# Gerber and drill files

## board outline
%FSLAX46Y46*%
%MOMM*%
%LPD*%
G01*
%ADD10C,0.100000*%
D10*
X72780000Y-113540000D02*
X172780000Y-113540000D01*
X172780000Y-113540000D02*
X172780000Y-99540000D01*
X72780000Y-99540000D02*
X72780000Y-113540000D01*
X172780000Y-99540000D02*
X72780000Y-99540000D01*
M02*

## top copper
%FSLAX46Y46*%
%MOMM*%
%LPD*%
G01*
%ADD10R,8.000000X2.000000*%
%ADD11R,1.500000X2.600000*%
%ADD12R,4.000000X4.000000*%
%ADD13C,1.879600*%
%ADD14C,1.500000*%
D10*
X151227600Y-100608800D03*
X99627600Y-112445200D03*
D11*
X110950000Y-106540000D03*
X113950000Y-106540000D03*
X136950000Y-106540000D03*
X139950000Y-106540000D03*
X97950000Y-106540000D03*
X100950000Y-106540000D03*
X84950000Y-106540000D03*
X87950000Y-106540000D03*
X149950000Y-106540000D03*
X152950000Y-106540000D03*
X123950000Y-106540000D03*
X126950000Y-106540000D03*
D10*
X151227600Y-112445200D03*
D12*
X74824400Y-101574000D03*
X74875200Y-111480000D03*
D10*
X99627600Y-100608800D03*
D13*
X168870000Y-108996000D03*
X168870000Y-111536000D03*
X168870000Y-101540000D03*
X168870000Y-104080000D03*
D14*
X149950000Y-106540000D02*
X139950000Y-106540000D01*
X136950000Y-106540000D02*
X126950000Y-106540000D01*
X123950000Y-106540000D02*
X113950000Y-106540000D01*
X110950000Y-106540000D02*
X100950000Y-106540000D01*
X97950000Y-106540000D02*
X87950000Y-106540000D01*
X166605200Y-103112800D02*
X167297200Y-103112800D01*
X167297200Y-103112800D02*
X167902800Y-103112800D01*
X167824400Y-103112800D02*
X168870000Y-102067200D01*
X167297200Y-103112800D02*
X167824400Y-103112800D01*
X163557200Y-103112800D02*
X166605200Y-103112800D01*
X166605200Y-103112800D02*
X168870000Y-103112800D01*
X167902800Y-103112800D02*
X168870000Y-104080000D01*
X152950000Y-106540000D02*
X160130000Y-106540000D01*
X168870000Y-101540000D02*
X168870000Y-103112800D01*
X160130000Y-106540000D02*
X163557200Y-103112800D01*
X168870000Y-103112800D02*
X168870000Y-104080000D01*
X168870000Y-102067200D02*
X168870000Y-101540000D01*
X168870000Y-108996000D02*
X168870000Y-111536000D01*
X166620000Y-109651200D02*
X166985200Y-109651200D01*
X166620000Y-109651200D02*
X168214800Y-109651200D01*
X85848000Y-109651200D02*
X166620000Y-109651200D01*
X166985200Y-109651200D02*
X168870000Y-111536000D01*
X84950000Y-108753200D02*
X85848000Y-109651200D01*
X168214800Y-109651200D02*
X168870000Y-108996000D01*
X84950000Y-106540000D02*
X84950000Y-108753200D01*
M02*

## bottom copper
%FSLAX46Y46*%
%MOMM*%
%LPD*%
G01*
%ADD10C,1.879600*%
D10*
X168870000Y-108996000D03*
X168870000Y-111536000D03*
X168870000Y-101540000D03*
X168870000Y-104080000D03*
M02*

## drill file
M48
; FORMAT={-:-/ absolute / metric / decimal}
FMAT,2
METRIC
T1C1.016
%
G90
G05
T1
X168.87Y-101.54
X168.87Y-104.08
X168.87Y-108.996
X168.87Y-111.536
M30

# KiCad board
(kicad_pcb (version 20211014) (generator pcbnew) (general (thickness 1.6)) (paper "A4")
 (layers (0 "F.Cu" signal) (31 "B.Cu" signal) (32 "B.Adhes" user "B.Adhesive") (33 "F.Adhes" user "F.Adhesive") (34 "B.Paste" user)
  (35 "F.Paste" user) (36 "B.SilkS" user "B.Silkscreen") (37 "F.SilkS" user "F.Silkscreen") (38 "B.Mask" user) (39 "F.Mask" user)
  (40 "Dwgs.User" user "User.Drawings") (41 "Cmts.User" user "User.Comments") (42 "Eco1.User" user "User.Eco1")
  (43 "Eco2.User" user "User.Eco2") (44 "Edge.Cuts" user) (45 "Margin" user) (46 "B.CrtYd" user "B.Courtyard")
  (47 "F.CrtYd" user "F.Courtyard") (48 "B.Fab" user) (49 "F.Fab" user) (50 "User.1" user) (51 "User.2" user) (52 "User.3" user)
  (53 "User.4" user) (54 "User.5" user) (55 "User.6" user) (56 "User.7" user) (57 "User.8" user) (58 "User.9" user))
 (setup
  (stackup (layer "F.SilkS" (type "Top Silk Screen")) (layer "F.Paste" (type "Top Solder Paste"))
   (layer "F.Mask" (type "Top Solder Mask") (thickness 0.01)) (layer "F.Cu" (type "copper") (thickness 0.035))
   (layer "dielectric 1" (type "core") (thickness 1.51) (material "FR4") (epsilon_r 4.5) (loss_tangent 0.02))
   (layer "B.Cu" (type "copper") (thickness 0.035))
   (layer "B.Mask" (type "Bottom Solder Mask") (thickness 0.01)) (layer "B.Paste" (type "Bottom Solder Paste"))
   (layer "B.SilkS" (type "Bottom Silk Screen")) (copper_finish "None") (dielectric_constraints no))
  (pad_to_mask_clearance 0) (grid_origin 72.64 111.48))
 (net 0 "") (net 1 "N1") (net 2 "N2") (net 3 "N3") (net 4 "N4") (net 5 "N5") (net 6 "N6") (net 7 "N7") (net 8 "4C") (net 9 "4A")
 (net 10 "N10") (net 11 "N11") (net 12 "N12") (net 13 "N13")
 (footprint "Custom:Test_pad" (layer "F.Cu") (at 151.2276 100.6088)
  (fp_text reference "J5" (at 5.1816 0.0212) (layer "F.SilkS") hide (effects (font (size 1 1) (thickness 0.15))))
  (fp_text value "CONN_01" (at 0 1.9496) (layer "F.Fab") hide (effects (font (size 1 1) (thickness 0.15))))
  (pad "1" smd rect (at 0 0) (size 8 2) (layers "F.Cu" "F.Mask") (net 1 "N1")))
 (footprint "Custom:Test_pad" (layer "F.Cu") (at 99.6276 112.4452)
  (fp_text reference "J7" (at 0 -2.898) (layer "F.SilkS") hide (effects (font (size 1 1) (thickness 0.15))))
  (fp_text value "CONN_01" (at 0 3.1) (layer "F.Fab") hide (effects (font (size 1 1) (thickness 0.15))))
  (pad "1" smd rect (at 0 0) (size 8 2) (layers "F.Cu" "F.Mask") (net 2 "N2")))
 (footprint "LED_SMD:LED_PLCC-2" (layer "F.Cu") (at 112.45 106.54)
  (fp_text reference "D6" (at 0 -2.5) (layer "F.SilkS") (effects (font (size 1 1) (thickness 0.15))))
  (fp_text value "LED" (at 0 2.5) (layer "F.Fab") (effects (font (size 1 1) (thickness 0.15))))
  (pad "1" smd rect (at -1.5 0) (size 1.5 2.6) (layers "F.Cu" "F.Paste" "F.Mask") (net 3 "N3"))
  (pad "2" smd rect (at 1.5 0) (size 1.5 2.6) (layers "F.Cu" "F.Paste" "F.Mask") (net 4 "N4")))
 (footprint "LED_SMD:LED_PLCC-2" (layer "F.Cu") (at 138.45 106.54)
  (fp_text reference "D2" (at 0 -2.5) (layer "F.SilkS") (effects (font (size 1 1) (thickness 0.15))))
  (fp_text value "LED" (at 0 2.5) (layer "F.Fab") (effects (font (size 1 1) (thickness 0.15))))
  (pad "1" smd rect (at -1.5 0) (size 1.5 2.6) (layers "F.Cu" "F.Paste" "F.Mask") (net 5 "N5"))
  (pad "2" smd rect (at 1.5 0) (size 1.5 2.6) (layers "F.Cu" "F.Paste" "F.Mask") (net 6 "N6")))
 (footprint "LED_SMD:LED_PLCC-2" (layer "F.Cu") (at 99.45 106.54)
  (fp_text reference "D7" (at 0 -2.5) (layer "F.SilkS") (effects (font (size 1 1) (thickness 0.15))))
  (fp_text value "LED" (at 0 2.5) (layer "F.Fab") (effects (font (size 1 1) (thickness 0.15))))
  (pad "1" smd rect (at -1.5 0) (size 1.5 2.6) (layers "F.Cu" "F.Paste" "F.Mask") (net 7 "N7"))
  (pad "2" smd rect (at 1.5 0) (size 1.5 2.6) (layers "F.Cu" "F.Paste" "F.Mask") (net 3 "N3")))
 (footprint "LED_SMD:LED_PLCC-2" (layer "F.Cu") (at 86.45 106.54)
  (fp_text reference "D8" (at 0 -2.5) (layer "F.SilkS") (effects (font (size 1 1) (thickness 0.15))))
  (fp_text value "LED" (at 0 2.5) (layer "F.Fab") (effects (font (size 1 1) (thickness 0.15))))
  (pad "1" smd rect (at -1.5 0) (size 1.5 2.6) (layers "F.Cu" "F.Paste" "F.Mask") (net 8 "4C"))
  (pad "2" smd rect (at 1.5 0) (size 1.5 2.6) (layers "F.Cu" "F.Paste" "F.Mask") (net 7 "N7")))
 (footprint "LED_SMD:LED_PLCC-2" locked (layer "F.Cu") (at 151.45 106.54)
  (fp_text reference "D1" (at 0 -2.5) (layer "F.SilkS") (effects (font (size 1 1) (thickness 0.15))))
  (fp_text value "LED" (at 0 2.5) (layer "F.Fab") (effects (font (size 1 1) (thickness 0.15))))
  (pad "1" smd rect locked (at -1.5 0) (size 1.5 2.6) (layers "F.Cu" "F.Paste" "F.Mask") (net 6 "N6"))
  (pad "2" smd rect locked (at 1.5 0) (size 1.5 2.6) (layers "F.Cu" "F.Paste" "F.Mask") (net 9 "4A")))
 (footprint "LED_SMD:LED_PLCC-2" (layer "F.Cu") (at 125.45 106.54)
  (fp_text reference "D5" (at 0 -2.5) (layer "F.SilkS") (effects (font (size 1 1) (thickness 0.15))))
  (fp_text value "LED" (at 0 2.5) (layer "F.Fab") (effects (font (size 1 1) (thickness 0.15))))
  (pad "1" smd rect (at -1.5 0) (size 1.5 2.6) (layers "F.Cu" "F.Paste" "F.Mask") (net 4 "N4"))
  (pad "2" smd rect (at 1.5 0) (size 1.5 2.6) (layers "F.Cu" "F.Paste" "F.Mask") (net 5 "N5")))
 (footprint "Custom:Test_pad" (layer "F.Cu") (at 151.2276 112.4452)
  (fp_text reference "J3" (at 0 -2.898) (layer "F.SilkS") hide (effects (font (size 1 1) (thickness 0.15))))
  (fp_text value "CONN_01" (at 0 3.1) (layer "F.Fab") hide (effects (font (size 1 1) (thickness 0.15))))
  (pad "1" smd rect (at 0 0) (size 8 2) (layers "F.Cu" "F.Mask") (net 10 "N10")))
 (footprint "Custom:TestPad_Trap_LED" (layer "F.Cu") (at 74.8244 101.574)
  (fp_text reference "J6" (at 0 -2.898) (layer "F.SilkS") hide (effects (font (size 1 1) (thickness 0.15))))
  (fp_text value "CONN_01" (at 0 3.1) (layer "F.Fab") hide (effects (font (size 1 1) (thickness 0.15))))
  (pad "1" smd rect (at 0 0) (size 4 4) (layers "F.Cu" "F.Mask") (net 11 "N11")))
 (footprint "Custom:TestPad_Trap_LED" (layer "F.Cu") (at 74.8752 111.48)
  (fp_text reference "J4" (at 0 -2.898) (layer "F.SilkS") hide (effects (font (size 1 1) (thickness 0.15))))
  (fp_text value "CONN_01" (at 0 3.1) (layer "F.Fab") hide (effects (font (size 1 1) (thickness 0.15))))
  (pad "1" smd rect (at 0 0) (size 4 4) (layers "F.Cu" "F.Mask") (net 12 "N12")))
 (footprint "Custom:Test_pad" (layer "F.Cu") (at 99.6276 100.6088)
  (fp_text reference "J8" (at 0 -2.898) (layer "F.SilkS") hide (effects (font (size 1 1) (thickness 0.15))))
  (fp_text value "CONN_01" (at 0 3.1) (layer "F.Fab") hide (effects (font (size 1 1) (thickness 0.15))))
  (pad "1" smd rect (at 0 0) (size 8 2) (layers "F.Cu" "F.Mask") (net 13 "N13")))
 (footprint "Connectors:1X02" (layer "B.Cu") (at 168.87 108.996 -90)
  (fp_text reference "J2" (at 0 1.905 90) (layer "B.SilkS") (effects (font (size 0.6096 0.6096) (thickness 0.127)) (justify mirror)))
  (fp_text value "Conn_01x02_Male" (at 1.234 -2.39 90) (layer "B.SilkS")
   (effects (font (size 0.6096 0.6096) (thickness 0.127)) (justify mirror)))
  (pad "1" thru_hole circle locked (at 0 0 270) (size 1.8796 1.8796) (drill 1.016) (layers *.Cu *.Mask) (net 8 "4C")
   (solder_mask_margin 0.1016))
  (pad "2" thru_hole circle locked (at 2.54 0 270) (size 1.8796 1.8796) (drill 1.016) (layers *.Cu *.Mask) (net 8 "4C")
   (solder_mask_margin 0.1016)))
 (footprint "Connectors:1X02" (layer "B.Cu") (at 168.87 101.54 -90)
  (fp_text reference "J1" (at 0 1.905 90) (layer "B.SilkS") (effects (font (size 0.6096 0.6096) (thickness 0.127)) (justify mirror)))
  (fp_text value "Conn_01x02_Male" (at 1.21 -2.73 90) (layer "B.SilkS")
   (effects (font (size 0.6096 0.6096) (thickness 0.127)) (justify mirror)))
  (pad "1" thru_hole circle locked (at 0 0 270) (size 1.8796 1.8796) (drill 1.016) (layers *.Cu *.Mask) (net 9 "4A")
   (solder_mask_margin 0.1016))
  (pad "2" thru_hole circle locked (at 2.54 0 270) (size 1.8796 1.8796) (drill 1.016) (layers *.Cu *.Mask) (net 9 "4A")
   (solder_mask_margin 0.1016)))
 (gr_line (start 72.78 113.54) (end 172.78 113.54) (layer "Edge.Cuts") (width 0.1))
 (gr_line (start 172.78 113.54) (end 172.78 99.54) (layer "Edge.Cuts") (width 0.1))
 (gr_line (start 72.78 99.54) (end 72.78 113.54) (layer "Edge.Cuts") (width 0.1))
 (gr_line (start 172.78 99.54) (end 72.78 99.54) (layer "Edge.Cuts") (width 0.1))
 (segment (start 149.95 106.54) (end 139.95 106.54) (width 1.5) (layer "F.Cu") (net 6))
 (segment (start 136.95 106.54) (end 126.95 106.54) (width 1.5) (layer "F.Cu") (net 5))
 (segment (start 123.95 106.54) (end 113.95 106.54) (width 1.5) (layer "F.Cu") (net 4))
 (segment (start 110.95 106.54) (end 100.95 106.54) (width 1.5) (layer "F.Cu") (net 3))
 (segment (start 97.95 106.54) (end 87.95 106.54) (width 1.5) (layer "F.Cu") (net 7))
 (segment (start 166.6052 103.1128) (end 167.2972 103.1128) (width 1.5) (layer "F.Cu") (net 9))
 (segment (start 167.2972 103.1128) (end 167.9028 103.1128) (width 1.5) (layer "F.Cu") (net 9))
 (segment (start 167.8244 103.1128) (end 168.87 102.0672) (width 1.5) (layer "F.Cu") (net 9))
 (segment (start 167.2972 103.1128) (end 167.8244 103.1128) (width 1.5) (layer "F.Cu") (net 9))
 (segment (start 163.5572 103.1128) (end 166.6052 103.1128) (width 1.5) (layer "F.Cu") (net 9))
 (segment (start 166.6052 103.1128) (end 168.87 103.1128) (width 1.5) (layer "F.Cu") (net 9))
 (segment (start 167.9028 103.1128) (end 168.87 104.08) (width 1.5) (layer "F.Cu") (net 9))
 (segment (start 152.95 106.54) (end 160.13 106.54) (width 1.5) (layer "F.Cu") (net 9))
 (segment (start 168.87 101.54) (end 168.87 103.1128) (width 1.5) (layer "F.Cu") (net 9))
 (segment (start 160.13 106.54) (end 163.5572 103.1128) (width 1.5) (layer "F.Cu") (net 9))
 (segment (start 168.87 103.1128) (end 168.87 104.08) (width 1.5) (layer "F.Cu") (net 9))
 (segment (start 168.87 102.0672) (end 168.87 101.54) (width 1.5) (layer "F.Cu") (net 9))
 (segment (start 168.87 108.996) (end 168.87 111.536) (width 1.5) (layer "F.Cu") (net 8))
 (segment (start 166.62 109.6512) (end 166.9852 109.6512) (width 1.5) (layer "F.Cu") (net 8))
 (segment (start 166.62 109.6512) (end 168.2148 109.6512) (width 1.5) (layer "F.Cu") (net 8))
 (segment (start 85.848 109.6512) (end 166.62 109.6512) (width 1.5) (layer "F.Cu") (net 8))
 (segment (start 166.9852 109.6512) (end 168.87 111.536) (width 1.5) (layer "F.Cu") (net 8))
 (segment (start 84.95 108.7532) (end 85.848 109.6512) (width 1.5) (layer "F.Cu") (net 8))
 (segment (start 168.2148 109.6512) (end 168.87 108.996) (width 1.5) (layer "F.Cu") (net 8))
 (segment (start 84.95 106.54) (end 84.95 108.7532) (width 1.5) (layer "F.Cu") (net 8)))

